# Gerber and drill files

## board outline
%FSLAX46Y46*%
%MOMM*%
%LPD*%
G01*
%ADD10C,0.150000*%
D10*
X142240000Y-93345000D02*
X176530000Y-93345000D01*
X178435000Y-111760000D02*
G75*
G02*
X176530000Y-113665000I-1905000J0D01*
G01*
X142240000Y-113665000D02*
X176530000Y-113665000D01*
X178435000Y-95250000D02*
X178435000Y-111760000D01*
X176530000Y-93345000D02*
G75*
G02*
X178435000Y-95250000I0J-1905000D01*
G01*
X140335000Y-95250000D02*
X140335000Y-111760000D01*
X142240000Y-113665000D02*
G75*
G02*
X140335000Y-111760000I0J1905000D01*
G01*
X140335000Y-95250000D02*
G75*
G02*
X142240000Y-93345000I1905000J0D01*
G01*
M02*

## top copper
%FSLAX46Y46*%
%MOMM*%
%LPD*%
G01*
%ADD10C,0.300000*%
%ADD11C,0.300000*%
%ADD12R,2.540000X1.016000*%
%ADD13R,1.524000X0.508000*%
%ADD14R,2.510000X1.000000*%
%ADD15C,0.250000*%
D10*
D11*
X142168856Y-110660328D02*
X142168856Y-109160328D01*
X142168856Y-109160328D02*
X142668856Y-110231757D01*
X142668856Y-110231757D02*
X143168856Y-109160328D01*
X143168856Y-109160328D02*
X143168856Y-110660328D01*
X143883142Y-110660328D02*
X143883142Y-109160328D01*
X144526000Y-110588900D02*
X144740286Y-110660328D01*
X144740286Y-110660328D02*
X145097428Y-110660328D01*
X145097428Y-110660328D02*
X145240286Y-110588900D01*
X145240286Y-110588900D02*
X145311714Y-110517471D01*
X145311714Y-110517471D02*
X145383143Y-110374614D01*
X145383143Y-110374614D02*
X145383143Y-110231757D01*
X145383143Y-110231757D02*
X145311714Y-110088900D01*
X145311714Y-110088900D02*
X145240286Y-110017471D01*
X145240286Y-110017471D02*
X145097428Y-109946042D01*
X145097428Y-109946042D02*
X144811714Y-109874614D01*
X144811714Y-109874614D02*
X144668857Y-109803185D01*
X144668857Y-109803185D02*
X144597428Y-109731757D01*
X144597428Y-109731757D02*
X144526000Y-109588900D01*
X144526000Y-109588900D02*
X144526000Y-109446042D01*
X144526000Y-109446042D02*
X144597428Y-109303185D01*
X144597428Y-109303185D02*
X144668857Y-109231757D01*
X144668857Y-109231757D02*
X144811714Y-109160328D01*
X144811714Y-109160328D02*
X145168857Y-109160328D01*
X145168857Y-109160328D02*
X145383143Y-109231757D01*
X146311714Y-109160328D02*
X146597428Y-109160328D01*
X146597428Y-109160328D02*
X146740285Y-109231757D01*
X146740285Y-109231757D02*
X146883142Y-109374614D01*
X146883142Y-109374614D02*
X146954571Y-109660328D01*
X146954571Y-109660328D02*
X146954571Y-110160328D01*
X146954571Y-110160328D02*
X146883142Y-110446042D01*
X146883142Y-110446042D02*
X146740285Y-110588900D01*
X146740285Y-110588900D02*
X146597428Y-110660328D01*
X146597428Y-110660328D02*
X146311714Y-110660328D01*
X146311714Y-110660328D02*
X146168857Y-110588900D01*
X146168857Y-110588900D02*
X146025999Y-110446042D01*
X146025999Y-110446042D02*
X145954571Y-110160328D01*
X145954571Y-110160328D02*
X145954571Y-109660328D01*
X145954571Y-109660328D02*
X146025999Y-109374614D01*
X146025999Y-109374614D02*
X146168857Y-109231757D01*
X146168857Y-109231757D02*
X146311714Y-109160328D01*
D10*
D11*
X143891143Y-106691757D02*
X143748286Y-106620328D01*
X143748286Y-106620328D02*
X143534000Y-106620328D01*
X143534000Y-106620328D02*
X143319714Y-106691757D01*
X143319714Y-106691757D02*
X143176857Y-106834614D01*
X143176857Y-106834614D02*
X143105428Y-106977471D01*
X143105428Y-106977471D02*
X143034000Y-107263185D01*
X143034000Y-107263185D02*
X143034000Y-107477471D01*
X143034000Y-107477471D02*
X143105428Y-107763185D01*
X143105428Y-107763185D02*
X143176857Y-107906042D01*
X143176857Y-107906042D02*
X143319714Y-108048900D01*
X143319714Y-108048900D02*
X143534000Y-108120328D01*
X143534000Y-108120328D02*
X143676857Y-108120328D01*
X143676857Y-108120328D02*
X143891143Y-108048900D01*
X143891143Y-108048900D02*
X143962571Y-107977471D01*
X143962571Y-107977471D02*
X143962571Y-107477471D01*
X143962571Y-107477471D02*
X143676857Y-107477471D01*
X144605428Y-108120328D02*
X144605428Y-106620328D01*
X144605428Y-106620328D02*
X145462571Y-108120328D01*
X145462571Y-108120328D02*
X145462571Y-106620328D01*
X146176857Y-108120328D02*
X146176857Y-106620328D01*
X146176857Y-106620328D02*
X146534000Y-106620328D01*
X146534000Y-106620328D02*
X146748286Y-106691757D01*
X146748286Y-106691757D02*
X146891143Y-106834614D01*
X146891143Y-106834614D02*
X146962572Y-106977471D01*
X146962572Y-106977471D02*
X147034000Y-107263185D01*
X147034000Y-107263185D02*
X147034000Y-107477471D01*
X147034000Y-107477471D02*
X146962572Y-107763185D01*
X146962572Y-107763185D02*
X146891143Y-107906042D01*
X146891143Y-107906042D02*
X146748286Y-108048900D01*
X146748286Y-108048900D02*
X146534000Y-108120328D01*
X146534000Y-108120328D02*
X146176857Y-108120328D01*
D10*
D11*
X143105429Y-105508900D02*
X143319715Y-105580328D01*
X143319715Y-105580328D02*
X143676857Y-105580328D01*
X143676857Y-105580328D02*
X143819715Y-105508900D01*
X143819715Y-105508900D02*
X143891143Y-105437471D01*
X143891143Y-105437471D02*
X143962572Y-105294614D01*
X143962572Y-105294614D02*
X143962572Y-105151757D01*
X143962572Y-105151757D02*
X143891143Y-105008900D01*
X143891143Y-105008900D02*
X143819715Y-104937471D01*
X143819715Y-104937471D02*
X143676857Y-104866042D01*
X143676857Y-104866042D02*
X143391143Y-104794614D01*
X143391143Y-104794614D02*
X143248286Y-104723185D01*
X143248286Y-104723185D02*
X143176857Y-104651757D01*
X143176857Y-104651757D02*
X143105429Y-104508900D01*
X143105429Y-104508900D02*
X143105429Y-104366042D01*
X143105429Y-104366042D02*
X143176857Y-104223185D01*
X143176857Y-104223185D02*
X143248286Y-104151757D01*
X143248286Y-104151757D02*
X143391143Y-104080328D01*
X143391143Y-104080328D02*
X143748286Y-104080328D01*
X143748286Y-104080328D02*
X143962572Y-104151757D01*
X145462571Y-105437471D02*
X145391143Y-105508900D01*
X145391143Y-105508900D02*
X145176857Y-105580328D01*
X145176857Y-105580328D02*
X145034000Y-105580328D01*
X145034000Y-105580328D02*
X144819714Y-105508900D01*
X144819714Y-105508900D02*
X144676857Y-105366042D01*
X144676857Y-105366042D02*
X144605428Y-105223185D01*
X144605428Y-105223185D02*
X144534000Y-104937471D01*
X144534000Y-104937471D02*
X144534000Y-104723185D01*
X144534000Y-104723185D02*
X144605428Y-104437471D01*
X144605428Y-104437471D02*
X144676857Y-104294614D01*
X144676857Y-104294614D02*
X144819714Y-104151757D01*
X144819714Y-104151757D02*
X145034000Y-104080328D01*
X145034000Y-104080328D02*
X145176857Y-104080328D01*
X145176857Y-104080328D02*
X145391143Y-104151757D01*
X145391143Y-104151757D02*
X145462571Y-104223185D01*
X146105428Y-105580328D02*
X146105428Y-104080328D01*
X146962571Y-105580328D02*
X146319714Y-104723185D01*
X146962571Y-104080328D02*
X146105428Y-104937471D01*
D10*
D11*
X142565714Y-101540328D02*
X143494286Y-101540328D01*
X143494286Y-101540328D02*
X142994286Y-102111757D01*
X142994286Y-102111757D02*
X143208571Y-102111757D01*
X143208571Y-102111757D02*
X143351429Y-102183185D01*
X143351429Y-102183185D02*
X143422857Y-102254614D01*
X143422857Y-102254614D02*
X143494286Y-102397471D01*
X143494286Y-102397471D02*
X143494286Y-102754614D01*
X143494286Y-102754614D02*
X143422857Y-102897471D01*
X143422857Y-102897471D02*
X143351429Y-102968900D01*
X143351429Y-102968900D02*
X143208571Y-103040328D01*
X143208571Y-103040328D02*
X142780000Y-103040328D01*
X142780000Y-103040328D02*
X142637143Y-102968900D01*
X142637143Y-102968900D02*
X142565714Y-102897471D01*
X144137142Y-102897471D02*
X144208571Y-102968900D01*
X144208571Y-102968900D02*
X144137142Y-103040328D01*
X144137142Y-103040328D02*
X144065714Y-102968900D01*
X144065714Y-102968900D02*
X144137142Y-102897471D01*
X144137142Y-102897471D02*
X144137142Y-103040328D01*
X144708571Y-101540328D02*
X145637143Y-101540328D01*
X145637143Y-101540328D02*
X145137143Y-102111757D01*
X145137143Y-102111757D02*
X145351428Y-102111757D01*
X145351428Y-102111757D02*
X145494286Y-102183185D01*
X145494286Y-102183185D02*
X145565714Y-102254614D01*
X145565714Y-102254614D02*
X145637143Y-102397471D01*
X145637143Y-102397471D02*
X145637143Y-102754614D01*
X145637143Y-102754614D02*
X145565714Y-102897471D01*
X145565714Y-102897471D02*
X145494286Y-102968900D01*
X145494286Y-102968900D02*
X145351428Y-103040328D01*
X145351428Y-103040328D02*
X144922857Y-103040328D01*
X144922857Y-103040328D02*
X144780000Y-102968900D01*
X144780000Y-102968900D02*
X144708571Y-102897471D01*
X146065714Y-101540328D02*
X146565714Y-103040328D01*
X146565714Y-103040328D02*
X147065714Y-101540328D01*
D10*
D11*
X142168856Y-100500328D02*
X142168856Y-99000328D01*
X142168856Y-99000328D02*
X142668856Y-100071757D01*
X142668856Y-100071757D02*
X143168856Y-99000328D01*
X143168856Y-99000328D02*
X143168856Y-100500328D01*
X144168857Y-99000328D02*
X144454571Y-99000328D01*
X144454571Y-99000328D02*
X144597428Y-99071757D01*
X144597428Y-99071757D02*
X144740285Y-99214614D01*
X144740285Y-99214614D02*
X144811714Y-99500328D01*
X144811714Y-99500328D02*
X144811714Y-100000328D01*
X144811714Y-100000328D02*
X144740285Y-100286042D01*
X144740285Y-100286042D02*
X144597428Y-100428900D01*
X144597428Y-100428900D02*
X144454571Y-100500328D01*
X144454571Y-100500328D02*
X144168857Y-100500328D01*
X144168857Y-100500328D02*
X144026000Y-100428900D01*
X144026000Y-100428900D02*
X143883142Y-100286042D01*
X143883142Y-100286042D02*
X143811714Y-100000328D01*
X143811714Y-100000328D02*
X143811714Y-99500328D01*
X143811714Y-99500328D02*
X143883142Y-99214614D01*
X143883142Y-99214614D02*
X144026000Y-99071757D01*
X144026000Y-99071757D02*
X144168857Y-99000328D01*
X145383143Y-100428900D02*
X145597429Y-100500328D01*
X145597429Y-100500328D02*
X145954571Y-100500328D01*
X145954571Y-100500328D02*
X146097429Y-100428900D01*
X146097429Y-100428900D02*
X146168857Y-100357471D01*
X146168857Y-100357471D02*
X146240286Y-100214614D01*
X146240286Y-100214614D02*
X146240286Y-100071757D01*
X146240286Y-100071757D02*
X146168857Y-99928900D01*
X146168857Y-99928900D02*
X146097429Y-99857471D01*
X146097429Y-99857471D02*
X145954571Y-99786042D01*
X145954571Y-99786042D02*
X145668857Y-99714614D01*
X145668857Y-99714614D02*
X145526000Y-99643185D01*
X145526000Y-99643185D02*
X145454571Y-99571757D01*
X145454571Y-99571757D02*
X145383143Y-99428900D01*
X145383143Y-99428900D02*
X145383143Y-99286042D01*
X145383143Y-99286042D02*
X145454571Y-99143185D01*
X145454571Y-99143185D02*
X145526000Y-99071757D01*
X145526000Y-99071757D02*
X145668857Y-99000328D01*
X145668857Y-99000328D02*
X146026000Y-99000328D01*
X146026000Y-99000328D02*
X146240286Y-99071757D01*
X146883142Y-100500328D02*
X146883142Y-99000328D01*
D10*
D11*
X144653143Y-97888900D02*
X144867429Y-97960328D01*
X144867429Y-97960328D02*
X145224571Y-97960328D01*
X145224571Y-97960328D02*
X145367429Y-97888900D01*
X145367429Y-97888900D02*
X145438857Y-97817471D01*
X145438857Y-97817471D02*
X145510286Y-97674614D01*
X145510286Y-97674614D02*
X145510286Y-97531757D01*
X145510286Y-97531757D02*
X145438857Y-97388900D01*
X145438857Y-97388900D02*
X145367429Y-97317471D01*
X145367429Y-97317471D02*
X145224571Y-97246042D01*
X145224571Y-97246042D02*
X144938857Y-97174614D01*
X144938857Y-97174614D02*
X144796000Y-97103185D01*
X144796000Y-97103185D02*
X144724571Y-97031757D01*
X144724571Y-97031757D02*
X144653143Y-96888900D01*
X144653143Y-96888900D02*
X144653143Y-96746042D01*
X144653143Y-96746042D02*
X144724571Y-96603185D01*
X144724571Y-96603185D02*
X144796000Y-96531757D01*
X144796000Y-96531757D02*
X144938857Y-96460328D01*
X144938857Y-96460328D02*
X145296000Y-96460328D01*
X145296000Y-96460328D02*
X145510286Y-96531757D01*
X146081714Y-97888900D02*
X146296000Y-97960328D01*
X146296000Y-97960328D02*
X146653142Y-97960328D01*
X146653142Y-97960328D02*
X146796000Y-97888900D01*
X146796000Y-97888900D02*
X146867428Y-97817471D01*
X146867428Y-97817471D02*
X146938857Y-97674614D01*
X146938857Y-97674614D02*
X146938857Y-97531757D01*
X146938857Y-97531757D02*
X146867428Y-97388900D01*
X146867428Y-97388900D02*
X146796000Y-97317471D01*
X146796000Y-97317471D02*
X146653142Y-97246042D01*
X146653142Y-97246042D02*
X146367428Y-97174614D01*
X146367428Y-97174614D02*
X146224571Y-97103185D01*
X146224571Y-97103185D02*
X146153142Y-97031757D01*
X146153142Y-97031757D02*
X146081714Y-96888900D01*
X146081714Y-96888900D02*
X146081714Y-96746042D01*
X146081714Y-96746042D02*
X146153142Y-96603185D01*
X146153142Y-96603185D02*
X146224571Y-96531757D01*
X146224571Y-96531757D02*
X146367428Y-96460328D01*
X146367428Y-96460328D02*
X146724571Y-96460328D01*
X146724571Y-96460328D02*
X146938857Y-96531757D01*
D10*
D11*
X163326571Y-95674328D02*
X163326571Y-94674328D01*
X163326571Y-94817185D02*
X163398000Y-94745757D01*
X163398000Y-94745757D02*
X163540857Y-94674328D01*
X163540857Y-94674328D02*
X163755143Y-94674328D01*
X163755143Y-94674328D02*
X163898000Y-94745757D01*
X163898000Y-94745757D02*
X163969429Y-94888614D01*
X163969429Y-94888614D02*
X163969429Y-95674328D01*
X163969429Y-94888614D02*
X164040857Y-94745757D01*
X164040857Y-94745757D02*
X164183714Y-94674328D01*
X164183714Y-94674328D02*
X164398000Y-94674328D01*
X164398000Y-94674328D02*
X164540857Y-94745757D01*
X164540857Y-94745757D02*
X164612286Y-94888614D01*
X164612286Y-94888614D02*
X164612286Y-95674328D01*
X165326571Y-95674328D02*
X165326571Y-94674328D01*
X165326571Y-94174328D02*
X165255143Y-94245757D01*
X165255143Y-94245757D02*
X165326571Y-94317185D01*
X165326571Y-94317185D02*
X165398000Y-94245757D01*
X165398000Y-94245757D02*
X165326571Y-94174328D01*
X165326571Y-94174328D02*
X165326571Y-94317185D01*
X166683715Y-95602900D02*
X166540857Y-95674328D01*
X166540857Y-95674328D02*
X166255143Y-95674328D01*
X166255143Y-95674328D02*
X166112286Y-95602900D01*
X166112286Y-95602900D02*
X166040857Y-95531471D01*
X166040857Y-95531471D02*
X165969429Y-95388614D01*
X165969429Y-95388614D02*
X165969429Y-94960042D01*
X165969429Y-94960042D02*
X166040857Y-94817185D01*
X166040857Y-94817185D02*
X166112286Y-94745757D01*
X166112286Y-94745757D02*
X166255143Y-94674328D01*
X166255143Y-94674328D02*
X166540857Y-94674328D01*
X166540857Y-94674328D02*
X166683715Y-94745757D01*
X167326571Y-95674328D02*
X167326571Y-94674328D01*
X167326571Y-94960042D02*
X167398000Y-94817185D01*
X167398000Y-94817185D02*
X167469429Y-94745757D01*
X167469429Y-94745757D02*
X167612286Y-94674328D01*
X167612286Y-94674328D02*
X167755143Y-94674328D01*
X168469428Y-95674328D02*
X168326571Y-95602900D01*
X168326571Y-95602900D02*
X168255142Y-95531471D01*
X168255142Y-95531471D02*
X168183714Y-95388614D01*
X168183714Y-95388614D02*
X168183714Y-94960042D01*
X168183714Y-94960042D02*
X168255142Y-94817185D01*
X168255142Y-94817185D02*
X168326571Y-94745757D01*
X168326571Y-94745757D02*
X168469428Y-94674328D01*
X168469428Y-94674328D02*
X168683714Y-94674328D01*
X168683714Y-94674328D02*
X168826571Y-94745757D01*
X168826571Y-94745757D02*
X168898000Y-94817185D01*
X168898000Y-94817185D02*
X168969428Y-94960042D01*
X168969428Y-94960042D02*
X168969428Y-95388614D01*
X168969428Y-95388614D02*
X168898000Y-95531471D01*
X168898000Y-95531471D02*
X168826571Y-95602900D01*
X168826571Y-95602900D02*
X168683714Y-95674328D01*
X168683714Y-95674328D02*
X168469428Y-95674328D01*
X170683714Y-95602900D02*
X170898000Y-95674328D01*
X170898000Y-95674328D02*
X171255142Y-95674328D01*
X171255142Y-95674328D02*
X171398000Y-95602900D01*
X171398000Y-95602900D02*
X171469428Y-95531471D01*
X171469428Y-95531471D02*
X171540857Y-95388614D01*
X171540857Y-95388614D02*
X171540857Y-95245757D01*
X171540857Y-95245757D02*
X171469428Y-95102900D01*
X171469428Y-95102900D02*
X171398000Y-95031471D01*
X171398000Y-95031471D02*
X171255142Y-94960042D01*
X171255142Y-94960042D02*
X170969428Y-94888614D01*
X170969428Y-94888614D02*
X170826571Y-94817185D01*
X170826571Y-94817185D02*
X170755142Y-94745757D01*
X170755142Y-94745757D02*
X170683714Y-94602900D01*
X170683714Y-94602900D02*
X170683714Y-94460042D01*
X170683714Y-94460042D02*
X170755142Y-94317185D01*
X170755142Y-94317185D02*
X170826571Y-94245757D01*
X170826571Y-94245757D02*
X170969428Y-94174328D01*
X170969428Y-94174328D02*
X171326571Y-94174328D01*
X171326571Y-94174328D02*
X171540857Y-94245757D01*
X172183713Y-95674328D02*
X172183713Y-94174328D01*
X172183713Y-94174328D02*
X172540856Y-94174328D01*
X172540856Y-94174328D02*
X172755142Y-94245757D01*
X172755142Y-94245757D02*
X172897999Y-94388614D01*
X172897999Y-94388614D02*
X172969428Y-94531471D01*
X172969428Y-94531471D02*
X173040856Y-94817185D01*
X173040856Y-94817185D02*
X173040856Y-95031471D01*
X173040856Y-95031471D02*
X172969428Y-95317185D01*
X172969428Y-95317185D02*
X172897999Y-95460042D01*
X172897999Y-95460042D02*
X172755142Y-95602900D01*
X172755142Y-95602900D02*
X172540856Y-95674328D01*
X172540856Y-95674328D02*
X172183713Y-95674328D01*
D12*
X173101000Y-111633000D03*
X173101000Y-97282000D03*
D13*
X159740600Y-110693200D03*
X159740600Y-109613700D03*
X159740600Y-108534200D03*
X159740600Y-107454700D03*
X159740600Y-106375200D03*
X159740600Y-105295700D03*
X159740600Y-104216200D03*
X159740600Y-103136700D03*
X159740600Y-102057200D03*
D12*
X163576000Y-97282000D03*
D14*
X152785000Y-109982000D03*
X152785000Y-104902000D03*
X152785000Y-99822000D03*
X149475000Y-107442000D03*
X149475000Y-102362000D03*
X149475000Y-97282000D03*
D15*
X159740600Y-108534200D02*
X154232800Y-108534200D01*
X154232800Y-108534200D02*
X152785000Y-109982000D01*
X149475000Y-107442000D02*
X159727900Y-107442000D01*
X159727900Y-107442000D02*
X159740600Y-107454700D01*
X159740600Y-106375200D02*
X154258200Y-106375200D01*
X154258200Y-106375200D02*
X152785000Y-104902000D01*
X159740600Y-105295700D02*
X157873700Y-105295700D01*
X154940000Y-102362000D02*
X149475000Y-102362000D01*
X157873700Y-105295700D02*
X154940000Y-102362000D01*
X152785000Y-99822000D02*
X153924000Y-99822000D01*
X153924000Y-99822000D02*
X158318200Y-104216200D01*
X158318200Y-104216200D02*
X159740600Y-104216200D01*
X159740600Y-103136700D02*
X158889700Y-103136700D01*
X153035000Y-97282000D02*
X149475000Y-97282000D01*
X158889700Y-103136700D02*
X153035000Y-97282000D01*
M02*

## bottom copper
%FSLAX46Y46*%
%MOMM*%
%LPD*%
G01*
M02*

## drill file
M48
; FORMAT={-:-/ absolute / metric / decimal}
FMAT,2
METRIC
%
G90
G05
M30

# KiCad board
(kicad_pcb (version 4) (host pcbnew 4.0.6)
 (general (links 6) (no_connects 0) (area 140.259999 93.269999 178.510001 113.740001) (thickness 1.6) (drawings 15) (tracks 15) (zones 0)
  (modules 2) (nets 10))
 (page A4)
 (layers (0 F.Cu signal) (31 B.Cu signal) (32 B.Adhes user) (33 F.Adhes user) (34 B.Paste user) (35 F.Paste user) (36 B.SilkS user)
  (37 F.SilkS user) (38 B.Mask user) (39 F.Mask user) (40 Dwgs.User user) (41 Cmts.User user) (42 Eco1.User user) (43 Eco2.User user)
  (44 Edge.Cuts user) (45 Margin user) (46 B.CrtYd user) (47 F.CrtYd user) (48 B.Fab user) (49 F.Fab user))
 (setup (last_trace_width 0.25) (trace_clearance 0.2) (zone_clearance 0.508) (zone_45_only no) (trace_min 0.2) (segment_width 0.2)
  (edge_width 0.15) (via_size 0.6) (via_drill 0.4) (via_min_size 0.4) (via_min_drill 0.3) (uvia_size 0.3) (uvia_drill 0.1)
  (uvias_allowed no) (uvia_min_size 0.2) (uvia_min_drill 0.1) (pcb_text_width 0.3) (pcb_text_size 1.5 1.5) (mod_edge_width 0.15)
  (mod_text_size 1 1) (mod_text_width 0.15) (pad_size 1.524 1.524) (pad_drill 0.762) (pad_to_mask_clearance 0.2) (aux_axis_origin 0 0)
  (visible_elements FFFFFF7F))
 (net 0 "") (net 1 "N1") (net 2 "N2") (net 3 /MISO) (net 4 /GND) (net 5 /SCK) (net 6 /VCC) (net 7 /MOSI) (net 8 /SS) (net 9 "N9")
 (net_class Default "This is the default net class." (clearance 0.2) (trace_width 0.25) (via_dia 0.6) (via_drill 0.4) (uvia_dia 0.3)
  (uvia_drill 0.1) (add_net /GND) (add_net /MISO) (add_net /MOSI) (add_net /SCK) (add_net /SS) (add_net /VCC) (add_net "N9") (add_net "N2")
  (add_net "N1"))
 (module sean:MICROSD (layer F.Cu) (at 168.148 104.902 90)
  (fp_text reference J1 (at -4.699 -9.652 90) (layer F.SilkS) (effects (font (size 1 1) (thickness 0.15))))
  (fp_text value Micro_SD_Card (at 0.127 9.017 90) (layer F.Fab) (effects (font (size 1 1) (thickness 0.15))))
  (pad SHEI smd rect (at -6.731 4.953 90) (size 1.016 2.54) (layers F.Cu F.Paste F.Mask))
  (pad SHEI smd rect (at 7.62 4.953 90) (size 1.016 2.54) (layers F.Cu F.Paste F.Mask))
  (pad 9 smd rect (at -5.7912 -8.4074 90) (size 0.508 1.524) (layers F.Cu F.Paste F.Mask) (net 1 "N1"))
  (pad 8 smd rect (at -4.7117 -8.4074 90) (size 0.508 1.524) (layers F.Cu F.Paste F.Mask) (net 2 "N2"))
  (pad 7 smd rect (at -3.6322 -8.4074 90) (size 0.508 1.524) (layers F.Cu F.Paste F.Mask) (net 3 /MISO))
  (pad 6 smd rect (at -2.5527 -8.4074 90) (size 0.508 1.524) (layers F.Cu F.Paste F.Mask) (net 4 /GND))
  (pad 5 smd rect (at -1.4732 -8.4074 90) (size 0.508 1.524) (layers F.Cu F.Paste F.Mask) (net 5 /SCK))
  (pad 4 smd rect (at -0.3937 -8.4074 90) (size 0.508 1.524) (layers F.Cu F.Paste F.Mask) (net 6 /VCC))
  (pad 3 smd rect (at 0.6858 -8.4074 90) (size 0.508 1.524) (layers F.Cu F.Paste F.Mask) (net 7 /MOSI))
  (pad 2 smd rect (at 1.7653 -8.4074 90) (size 0.508 1.524) (layers F.Cu F.Paste F.Mask) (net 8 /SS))
  (pad 1 smd rect (at 2.8448 -8.4074 90) (size 0.508 1.524) (layers F.Cu F.Paste F.Mask) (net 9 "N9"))
  (pad SHEI smd rect (at 7.62 -4.572 90) (size 1.016 2.54) (layers F.Cu F.Paste F.Mask)))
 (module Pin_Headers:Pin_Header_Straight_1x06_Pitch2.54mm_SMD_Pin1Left (layer F.Cu) (at 151.13 103.632 180)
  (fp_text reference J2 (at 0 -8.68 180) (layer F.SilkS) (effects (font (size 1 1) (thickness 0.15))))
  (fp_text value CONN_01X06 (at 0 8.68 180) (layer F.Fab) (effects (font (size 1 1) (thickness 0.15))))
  (pad 1 smd rect (at -1.655 -6.35 180) (size 2.51 1) (layers F.Cu F.Paste F.Mask) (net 3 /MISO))
  (pad 3 smd rect (at -1.655 -1.27 180) (size 2.51 1) (layers F.Cu F.Paste F.Mask) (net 5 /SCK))
  (pad 5 smd rect (at -1.655 3.81 180) (size 2.51 1) (layers F.Cu F.Paste F.Mask) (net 7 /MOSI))
  (pad 2 smd rect (at 1.655 -3.81 180) (size 2.51 1) (layers F.Cu F.Paste F.Mask) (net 4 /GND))
  (pad 4 smd rect (at 1.655 1.27 180) (size 2.51 1) (layers F.Cu F.Paste F.Mask) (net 6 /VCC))
  (pad 6 smd rect (at 1.655 6.35 180) (size 2.51 1) (layers F.Cu F.Paste F.Mask) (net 8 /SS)))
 (gr_line (start 142.24 93.345) (end 176.53 93.345) (angle 90) (layer Edge.Cuts) (width 0.15))
 (gr_arc (start 176.53 111.76) (end 178.435 111.76) (angle 90) (layer Edge.Cuts) (width 0.15))
 (gr_line (start 142.24 113.665) (end 176.53 113.665) (angle 90) (layer Edge.Cuts) (width 0.15))
 (gr_line (start 178.435 95.25) (end 178.435 111.76) (angle 90) (layer Edge.Cuts) (width 0.15))
 (gr_arc (start 176.53 95.25) (end 176.53 93.345) (angle 90) (layer Edge.Cuts) (width 0.15))
 (gr_line (start 140.335 95.25) (end 140.335 111.76) (angle 90) (layer Edge.Cuts) (width 0.15))
 (gr_arc (start 142.24 111.76) (end 142.24 113.665) (angle 90) (layer Edge.Cuts) (width 0.15))
 (gr_arc (start 142.24 95.25) (end 140.335 95.25) (angle 90) (layer Edge.Cuts) (width 0.15))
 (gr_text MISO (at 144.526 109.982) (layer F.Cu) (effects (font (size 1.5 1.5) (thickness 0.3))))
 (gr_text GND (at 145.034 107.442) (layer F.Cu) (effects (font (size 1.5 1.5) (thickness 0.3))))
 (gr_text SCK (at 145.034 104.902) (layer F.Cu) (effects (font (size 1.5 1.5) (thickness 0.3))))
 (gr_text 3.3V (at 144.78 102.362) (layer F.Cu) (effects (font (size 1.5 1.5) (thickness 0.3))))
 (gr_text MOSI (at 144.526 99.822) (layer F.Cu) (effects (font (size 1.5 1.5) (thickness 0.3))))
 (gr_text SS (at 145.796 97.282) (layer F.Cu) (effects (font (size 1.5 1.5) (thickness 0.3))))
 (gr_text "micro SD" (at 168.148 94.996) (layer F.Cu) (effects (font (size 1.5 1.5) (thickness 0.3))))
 (segment (start 159.7406 108.5342) (end 154.2328 108.5342) (width 0.25) (layer F.Cu) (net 3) (status 400000))
 (segment (start 154.2328 108.5342) (end 152.785 109.982) (width 0.25) (layer F.Cu) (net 3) (status 800000))
 (segment (start 149.475 107.442) (end 159.7279 107.442) (width 0.25) (layer F.Cu) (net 4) (status C00000))
 (segment (start 159.7279 107.442) (end 159.7406 107.4547) (width 0.25) (layer F.Cu) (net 4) (status C00000))
 (segment (start 159.7406 106.3752) (end 154.2582 106.3752) (width 0.25) (layer F.Cu) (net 5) (status 400000))
 (segment (start 154.2582 106.3752) (end 152.785 104.902) (width 0.25) (layer F.Cu) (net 5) (status 800000))
 (segment (start 159.7406 105.2957) (end 157.8737 105.2957) (width 0.25) (layer F.Cu) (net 6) (status 400000))
 (segment (start 154.94 102.362) (end 149.475 102.362) (width 0.25) (layer F.Cu) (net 6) (status 800000))
 (segment (start 157.8737 105.2957) (end 154.94 102.362) (width 0.25) (layer F.Cu) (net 6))
 (segment (start 152.785 99.822) (end 153.924 99.822) (width 0.25) (layer F.Cu) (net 7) (status C00000))
 (segment (start 153.924 99.822) (end 158.3182 104.2162) (width 0.25) (layer F.Cu) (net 7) (status 400000))
 (segment (start 158.3182 104.2162) (end 159.7406 104.2162) (width 0.25) (layer F.Cu) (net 7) (status 800000))
 (segment (start 159.7406 103.1367) (end 158.8897 103.1367) (width 0.25) (layer F.Cu) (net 8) (status 400000))
 (segment (start 153.035 97.282) (end 149.475 97.282) (width 0.25) (layer F.Cu) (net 8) (status 800000))
 (segment (start 158.8897 103.1367) (end 153.035 97.282) (width 0.25) (layer F.Cu) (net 8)))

